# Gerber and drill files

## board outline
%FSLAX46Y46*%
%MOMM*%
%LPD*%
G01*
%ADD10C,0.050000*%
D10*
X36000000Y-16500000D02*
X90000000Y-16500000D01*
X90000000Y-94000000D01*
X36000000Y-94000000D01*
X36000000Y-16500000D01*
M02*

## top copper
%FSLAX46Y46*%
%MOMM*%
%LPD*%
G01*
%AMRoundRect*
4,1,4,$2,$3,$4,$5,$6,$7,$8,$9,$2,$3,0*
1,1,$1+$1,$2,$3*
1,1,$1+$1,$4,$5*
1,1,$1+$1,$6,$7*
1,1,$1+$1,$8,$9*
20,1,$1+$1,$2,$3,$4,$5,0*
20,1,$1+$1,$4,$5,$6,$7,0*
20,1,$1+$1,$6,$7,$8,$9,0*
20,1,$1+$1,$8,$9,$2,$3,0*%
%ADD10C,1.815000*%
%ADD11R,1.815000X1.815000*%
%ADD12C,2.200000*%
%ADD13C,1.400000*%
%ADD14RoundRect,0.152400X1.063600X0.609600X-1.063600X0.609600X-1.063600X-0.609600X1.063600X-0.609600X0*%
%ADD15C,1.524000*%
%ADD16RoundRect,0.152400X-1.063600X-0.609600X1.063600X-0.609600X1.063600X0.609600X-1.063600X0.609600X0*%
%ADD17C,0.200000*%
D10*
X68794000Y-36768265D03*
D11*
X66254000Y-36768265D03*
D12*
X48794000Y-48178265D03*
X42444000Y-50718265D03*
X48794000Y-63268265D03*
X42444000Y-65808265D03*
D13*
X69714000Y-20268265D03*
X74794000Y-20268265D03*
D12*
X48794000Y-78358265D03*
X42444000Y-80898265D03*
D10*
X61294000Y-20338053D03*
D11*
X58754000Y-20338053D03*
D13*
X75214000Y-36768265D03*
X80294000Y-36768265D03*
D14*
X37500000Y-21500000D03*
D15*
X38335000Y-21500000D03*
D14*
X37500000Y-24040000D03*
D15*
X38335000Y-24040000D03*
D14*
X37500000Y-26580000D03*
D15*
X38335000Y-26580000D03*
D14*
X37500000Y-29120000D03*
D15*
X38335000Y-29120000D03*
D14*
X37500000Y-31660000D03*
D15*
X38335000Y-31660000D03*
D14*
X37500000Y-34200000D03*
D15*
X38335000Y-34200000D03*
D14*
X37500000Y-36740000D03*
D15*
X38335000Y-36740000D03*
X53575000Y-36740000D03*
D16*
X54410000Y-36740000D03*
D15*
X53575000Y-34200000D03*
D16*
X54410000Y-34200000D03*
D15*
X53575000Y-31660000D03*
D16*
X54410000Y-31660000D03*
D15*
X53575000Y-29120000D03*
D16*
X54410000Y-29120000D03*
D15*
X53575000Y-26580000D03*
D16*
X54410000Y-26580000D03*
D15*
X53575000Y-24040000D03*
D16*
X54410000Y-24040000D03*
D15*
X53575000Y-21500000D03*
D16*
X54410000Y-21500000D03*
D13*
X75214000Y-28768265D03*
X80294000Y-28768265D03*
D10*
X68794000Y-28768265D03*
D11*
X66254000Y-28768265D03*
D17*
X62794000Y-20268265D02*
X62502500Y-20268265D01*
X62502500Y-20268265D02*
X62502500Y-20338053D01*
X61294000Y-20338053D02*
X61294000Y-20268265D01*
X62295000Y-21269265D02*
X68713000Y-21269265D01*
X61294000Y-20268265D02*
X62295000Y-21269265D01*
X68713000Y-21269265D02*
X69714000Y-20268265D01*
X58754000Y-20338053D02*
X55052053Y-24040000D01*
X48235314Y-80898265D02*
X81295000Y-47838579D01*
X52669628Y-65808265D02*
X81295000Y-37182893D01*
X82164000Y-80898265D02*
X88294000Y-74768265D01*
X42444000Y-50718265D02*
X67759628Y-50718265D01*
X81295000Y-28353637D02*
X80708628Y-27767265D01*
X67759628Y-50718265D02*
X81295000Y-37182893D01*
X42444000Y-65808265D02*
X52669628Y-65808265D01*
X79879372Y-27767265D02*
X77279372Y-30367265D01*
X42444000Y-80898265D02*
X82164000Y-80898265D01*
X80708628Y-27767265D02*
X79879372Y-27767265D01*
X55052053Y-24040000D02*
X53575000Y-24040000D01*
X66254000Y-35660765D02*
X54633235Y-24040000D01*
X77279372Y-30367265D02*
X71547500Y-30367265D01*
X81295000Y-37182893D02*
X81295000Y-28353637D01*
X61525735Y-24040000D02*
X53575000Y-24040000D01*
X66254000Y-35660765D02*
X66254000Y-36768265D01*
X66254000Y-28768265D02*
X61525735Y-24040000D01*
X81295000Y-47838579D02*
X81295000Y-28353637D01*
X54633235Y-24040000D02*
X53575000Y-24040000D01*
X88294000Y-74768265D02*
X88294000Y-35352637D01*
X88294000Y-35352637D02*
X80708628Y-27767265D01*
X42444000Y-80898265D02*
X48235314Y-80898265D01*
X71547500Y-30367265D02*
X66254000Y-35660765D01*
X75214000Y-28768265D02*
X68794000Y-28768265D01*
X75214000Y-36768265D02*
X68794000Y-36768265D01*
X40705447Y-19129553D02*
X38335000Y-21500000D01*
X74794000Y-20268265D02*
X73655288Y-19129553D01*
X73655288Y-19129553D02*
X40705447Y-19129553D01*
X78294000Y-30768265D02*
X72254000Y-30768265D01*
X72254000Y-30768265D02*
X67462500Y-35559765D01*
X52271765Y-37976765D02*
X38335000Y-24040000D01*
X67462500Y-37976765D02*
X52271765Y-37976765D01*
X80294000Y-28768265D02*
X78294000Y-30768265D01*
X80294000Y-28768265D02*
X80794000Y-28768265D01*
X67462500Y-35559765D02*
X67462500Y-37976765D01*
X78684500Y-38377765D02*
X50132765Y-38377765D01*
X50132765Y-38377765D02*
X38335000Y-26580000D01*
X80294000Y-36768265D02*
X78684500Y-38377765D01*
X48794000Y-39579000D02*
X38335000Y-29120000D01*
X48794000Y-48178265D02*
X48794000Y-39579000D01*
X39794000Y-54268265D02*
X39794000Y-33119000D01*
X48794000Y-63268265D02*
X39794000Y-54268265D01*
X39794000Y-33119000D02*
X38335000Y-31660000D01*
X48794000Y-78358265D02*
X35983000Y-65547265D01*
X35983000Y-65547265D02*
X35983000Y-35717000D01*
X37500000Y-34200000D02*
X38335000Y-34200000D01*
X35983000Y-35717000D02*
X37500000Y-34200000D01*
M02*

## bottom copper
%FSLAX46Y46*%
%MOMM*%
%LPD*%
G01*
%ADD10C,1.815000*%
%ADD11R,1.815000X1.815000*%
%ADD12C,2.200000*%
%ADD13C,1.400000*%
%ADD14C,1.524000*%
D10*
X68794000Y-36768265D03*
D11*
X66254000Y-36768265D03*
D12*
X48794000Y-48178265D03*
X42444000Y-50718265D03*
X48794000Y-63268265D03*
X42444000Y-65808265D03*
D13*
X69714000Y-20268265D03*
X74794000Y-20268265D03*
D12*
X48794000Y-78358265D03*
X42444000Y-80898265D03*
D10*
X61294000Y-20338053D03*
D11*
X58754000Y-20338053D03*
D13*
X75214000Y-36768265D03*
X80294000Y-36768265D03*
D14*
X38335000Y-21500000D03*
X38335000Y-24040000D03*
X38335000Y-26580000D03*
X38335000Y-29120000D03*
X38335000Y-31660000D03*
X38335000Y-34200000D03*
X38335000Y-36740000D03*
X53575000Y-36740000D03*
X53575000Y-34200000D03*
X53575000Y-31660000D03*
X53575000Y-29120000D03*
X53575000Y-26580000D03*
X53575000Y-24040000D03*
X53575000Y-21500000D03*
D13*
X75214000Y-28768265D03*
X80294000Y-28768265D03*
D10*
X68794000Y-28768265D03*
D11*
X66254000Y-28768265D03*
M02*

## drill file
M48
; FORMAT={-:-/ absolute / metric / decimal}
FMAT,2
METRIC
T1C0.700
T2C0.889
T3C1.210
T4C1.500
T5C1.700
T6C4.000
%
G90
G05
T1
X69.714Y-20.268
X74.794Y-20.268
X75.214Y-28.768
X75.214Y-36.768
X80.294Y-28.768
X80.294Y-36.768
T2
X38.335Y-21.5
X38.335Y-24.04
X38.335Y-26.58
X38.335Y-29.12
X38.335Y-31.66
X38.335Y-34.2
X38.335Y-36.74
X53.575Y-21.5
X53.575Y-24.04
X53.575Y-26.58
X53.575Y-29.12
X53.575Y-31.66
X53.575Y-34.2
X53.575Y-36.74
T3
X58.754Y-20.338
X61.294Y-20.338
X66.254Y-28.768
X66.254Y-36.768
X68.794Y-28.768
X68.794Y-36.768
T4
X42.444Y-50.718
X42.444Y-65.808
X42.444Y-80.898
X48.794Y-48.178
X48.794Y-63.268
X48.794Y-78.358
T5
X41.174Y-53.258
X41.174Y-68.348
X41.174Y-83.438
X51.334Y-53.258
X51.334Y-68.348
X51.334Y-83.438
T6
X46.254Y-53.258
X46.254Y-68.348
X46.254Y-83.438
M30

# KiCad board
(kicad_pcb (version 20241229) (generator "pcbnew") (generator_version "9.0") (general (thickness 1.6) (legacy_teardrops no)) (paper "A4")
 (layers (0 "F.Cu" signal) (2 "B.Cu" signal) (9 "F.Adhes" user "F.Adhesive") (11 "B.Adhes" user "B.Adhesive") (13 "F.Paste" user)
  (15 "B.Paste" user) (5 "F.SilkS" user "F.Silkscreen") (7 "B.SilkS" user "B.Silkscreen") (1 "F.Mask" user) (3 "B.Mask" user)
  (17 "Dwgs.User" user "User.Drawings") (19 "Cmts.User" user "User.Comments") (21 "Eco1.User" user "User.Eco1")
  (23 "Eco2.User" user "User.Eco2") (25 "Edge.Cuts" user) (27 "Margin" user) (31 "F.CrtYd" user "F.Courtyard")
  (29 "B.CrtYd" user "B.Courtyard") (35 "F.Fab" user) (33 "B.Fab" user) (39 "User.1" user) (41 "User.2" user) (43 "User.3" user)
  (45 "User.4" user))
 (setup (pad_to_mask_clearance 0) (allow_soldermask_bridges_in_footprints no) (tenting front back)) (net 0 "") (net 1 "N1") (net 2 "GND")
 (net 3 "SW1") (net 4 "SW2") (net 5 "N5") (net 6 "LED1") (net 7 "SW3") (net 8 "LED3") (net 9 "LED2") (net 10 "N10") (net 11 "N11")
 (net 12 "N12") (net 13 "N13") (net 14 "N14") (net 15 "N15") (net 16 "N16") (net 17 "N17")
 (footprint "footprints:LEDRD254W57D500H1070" (layer "F.Cu") (at 67.524 36.768265)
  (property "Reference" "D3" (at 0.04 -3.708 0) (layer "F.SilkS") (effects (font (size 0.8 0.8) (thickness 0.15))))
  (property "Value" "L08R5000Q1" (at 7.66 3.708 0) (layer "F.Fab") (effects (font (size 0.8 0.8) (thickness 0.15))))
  (pad "A" thru_hole circle (at 1.27 0) (size 1.815 1.815) (drill 1.21) (layers "*.Cu" "*.Mask") (remove_unused_layers no) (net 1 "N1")
   (solder_mask_margin 0.102))
  (pad "C" thru_hole rect (at -1.27 0) (size 1.815 1.815) (drill 1.21) (layers "*.Cu" "*.Mask") (remove_unused_layers no) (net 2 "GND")
   (solder_mask_margin 0.102)))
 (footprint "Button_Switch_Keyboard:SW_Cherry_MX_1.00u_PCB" (layer "F.Cu") (at 48.794 48.178265)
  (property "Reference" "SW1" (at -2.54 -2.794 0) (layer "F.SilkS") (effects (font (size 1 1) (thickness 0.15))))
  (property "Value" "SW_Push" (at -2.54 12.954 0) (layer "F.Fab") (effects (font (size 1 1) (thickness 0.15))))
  (pad "" np_thru_hole circle (at -7.62 5.08) (size 1.7 1.7) (drill 1.7) (layers "*.Cu" "*.Mask"))
  (pad "" np_thru_hole circle (at -2.54 5.08) (size 4 4) (drill 4) (layers "*.Cu" "*.Mask"))
  (pad "" np_thru_hole circle (at 2.54 5.08) (size 1.7 1.7) (drill 1.7) (layers "*.Cu" "*.Mask"))
  (pad "1" thru_hole circle (at 0 0) (size 2.2 2.2) (drill 1.5) (layers "*.Cu" "*.Mask") (remove_unused_layers no) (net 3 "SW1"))
  (pad "2" thru_hole circle (at -6.35 2.54) (size 2.2 2.2) (drill 1.5) (layers "*.Cu" "*.Mask") (remove_unused_layers no) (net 2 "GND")))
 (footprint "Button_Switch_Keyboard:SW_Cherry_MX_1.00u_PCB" (layer "F.Cu") (at 48.794 63.268265)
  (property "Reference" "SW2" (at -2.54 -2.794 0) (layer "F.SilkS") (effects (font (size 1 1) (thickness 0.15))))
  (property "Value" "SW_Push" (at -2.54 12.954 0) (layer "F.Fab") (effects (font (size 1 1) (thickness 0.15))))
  (pad "" np_thru_hole circle (at -7.62 5.08) (size 1.7 1.7) (drill 1.7) (layers "*.Cu" "*.Mask"))
  (pad "" np_thru_hole circle (at -2.54 5.08) (size 4 4) (drill 4) (layers "*.Cu" "*.Mask"))
  (pad "" np_thru_hole circle (at 2.54 5.08) (size 1.7 1.7) (drill 1.7) (layers "*.Cu" "*.Mask"))
  (pad "1" thru_hole circle (at 0 0) (size 2.2 2.2) (drill 1.5) (layers "*.Cu" "*.Mask") (remove_unused_layers no) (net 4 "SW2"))
  (pad "2" thru_hole circle (at -6.35 2.54) (size 2.2 2.2) (drill 1.5) (layers "*.Cu" "*.Mask") (remove_unused_layers no) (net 2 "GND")))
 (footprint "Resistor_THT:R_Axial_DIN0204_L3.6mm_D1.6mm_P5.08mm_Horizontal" (layer "F.Cu") (at 69.714 20.268265)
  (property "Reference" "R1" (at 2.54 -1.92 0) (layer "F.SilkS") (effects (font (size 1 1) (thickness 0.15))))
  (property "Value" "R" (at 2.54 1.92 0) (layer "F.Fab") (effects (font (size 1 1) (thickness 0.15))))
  (pad "1" thru_hole circle (at 0 0) (size 1.4 1.4) (drill 0.7) (layers "*.Cu" "*.Mask") (remove_unused_layers no) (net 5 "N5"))
  (pad "2" thru_hole circle (at 5.08 0) (size 1.4 1.4) (drill 0.7) (layers "*.Cu" "*.Mask") (remove_unused_layers no) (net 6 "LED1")))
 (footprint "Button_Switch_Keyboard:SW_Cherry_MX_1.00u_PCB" (layer "F.Cu") (at 48.794 78.358265)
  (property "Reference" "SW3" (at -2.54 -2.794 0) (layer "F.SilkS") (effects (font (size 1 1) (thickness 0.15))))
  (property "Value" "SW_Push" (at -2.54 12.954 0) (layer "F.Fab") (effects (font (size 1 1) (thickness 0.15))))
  (pad "" np_thru_hole circle (at -7.62 5.08) (size 1.7 1.7) (drill 1.7) (layers "*.Cu" "*.Mask"))
  (pad "" np_thru_hole circle (at -2.54 5.08) (size 4 4) (drill 4) (layers "*.Cu" "*.Mask"))
  (pad "" np_thru_hole circle (at 2.54 5.08) (size 1.7 1.7) (drill 1.7) (layers "*.Cu" "*.Mask"))
  (pad "1" thru_hole circle (at 0 0) (size 2.2 2.2) (drill 1.5) (layers "*.Cu" "*.Mask") (remove_unused_layers no) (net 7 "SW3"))
  (pad "2" thru_hole circle (at -6.35 2.54) (size 2.2 2.2) (drill 1.5) (layers "*.Cu" "*.Mask") (remove_unused_layers no) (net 2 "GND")))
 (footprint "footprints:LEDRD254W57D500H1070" (layer "F.Cu") (at 60.024 20.338053)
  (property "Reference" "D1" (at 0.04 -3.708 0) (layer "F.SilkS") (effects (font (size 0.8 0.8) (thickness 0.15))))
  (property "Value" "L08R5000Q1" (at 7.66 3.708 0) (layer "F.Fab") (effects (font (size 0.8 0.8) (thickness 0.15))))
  (pad "A" thru_hole circle (at 1.27 0) (size 1.815 1.815) (drill 1.21) (layers "*.Cu" "*.Mask") (remove_unused_layers no) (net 5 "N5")
   (solder_mask_margin 0.102))
  (pad "C" thru_hole rect (at -1.27 0) (size 1.815 1.815) (drill 1.21) (layers "*.Cu" "*.Mask") (remove_unused_layers no) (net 2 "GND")
   (solder_mask_margin 0.102)))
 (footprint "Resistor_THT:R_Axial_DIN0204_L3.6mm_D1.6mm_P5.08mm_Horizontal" (layer "F.Cu") (at 75.214 36.768265)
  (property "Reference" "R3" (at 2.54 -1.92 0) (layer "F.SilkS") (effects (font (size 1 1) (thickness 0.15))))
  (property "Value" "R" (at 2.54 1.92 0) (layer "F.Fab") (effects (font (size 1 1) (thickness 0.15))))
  (pad "1" thru_hole circle (at 0 0) (size 1.4 1.4) (drill 0.7) (layers "*.Cu" "*.Mask") (remove_unused_layers no) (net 1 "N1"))
  (pad "2" thru_hole circle (at 5.08 0) (size 1.4 1.4) (drill 0.7) (layers "*.Cu" "*.Mask") (remove_unused_layers no) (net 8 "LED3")))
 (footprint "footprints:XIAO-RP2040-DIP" (layer "F.Cu") (at 45.955 29.12)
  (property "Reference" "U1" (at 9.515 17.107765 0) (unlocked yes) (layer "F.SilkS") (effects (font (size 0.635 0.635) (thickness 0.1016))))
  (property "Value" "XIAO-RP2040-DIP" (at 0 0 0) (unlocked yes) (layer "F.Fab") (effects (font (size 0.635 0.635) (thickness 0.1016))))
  (pad "1" smd roundrect (at -8.455 -7.62 180) (size 2.432 1.524) (layers "F.Cu" "F.Mask") (roundrect_rratio 0.1) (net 6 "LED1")
   (thermal_bridge_angle 45))
  (pad "1" thru_hole circle (at -7.62 -7.62 180) (size 1.524 1.524) (drill 0.889) (layers "*.Cu" "*.Mask") (remove_unused_layers no)
   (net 6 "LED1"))
  (pad "2" smd roundrect (at -8.455 -5.08 180) (size 2.432 1.524) (layers "F.Cu" "F.Mask") (roundrect_rratio 0.1) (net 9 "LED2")
   (thermal_bridge_angle 45))
  (pad "2" thru_hole circle (at -7.62 -5.08 180) (size 1.524 1.524) (drill 0.889) (layers "*.Cu" "*.Mask") (remove_unused_layers no)
   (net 9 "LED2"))
  (pad "3" smd roundrect (at -8.455 -2.54 180) (size 2.432 1.524) (layers "F.Cu" "F.Mask") (roundrect_rratio 0.1) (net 8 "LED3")
   (thermal_bridge_angle 45))
  (pad "3" thru_hole circle (at -7.62 -2.54 180) (size 1.524 1.524) (drill 0.889) (layers "*.Cu" "*.Mask") (remove_unused_layers no)
   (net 8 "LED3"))
  (pad "4" smd roundrect (at -8.455 0 180) (size 2.432 1.524) (layers "F.Cu" "F.Mask") (roundrect_rratio 0.1) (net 3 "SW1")
   (thermal_bridge_angle 45))
  (pad "4" thru_hole circle (at -7.62 0 180) (size 1.524 1.524) (drill 0.889) (layers "*.Cu" "*.Mask") (remove_unused_layers no)
   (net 3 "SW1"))
  (pad "5" smd roundrect (at -8.455 2.54 180) (size 2.432 1.524) (layers "F.Cu" "F.Mask") (roundrect_rratio 0.1) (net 4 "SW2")
   (thermal_bridge_angle 45))
  (pad "5" thru_hole circle (at -7.62 2.54 180) (size 1.524 1.524) (drill 0.889) (layers "*.Cu" "*.Mask") (remove_unused_layers no)
   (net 4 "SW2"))
  (pad "6" smd roundrect (at -8.455 5.08 180) (size 2.432 1.524) (layers "F.Cu" "F.Mask") (roundrect_rratio 0.1) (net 7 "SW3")
   (thermal_bridge_angle 45))
  (pad "6" thru_hole circle (at -7.62 5.08 180) (size 1.524 1.524) (drill 0.889) (layers "*.Cu" "*.Mask") (remove_unused_layers no)
   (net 7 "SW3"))
  (pad "7" smd roundrect (at -8.455 7.62 180) (size 2.432 1.524) (layers "F.Cu" "F.Mask") (roundrect_rratio 0.1) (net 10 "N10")
   (thermal_bridge_angle 45))
  (pad "7" thru_hole circle (at -7.62 7.62 180) (size 1.524 1.524) (drill 0.889) (layers "*.Cu" "*.Mask") (remove_unused_layers no)
   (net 10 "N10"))
  (pad "8" thru_hole circle (at 7.62 7.62) (size 1.524 1.524) (drill 0.889) (layers "*.Cu" "*.Mask") (remove_unused_layers no)
   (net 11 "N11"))
  (pad "8" smd roundrect (at 8.455 7.62) (size 2.432 1.524) (layers "F.Cu" "F.Mask") (roundrect_rratio 0.1) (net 11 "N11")
   (thermal_bridge_angle 45))
  (pad "9" thru_hole circle (at 7.62 5.08) (size 1.524 1.524) (drill 0.889) (layers "*.Cu" "*.Mask") (remove_unused_layers no)
   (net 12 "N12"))
  (pad "9" smd roundrect (at 8.455 5.08) (size 2.432 1.524) (layers "F.Cu" "F.Mask") (roundrect_rratio 0.1) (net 12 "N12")
   (thermal_bridge_angle 45))
  (pad "10" thru_hole circle (at 7.62 2.54) (size 1.524 1.524) (drill 0.889) (layers "*.Cu" "*.Mask") (remove_unused_layers no)
   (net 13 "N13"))
  (pad "10" smd roundrect (at 8.455 2.54) (size 2.432 1.524) (layers "F.Cu" "F.Mask") (roundrect_rratio 0.1) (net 13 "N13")
   (thermal_bridge_angle 45))
  (pad "11" thru_hole circle (at 7.62 0) (size 1.524 1.524) (drill 0.889) (layers "*.Cu" "*.Mask") (remove_unused_layers no) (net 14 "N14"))
  (pad "11" smd roundrect (at 8.455 0) (size 2.432 1.524) (layers "F.Cu" "F.Mask") (roundrect_rratio 0.1) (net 14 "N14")
   (thermal_bridge_angle 45))
  (pad "12" thru_hole circle (at 7.62 -2.54) (size 1.524 1.524) (drill 0.889) (layers "*.Cu" "*.Mask") (remove_unused_layers no)
   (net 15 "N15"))
  (pad "12" smd roundrect (at 8.455 -2.54) (size 2.432 1.524) (layers "F.Cu" "F.Mask") (roundrect_rratio 0.1) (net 15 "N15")
   (thermal_bridge_angle 45))
  (pad "13" thru_hole circle (at 7.62 -5.08) (size 1.524 1.524) (drill 0.889) (layers "*.Cu" "*.Mask") (remove_unused_layers no)
   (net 2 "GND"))
  (pad "13" smd roundrect (at 8.455 -5.08) (size 2.432 1.524) (layers "F.Cu" "F.Mask") (roundrect_rratio 0.1) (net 2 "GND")
   (thermal_bridge_angle 45))
  (pad "14" thru_hole circle (at 7.62 -7.62) (size 1.524 1.524) (drill 0.889) (layers "*.Cu" "*.Mask") (remove_unused_layers no)
   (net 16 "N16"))
  (pad "14" smd roundrect (at 8.455 -7.62) (size 2.432 1.524) (layers "F.Cu" "F.Mask") (roundrect_rratio 0.1) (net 16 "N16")
   (thermal_bridge_angle 45)))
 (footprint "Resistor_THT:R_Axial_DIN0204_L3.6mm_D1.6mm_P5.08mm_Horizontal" (layer "F.Cu") (at 75.214 28.768265)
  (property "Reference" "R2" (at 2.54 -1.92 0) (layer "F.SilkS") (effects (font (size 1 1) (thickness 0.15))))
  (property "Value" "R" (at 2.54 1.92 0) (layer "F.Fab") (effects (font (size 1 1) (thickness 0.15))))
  (pad "1" thru_hole circle (at 0 0) (size 1.4 1.4) (drill 0.7) (layers "*.Cu" "*.Mask") (remove_unused_layers no) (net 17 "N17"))
  (pad "2" thru_hole circle (at 5.08 0) (size 1.4 1.4) (drill 0.7) (layers "*.Cu" "*.Mask") (remove_unused_layers no) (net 9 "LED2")))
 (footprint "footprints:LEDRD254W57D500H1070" (layer "F.Cu") (at 67.524 28.768265)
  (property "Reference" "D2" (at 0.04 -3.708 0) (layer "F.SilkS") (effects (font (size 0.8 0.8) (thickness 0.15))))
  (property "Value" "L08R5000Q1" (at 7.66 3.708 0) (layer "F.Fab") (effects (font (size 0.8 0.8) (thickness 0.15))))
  (pad "A" thru_hole circle (at 1.27 0) (size 1.815 1.815) (drill 1.21) (layers "*.Cu" "*.Mask") (remove_unused_layers no) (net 17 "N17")
   (solder_mask_margin 0.102))
  (pad "C" thru_hole rect (at -1.27 0) (size 1.815 1.815) (drill 1.21) (layers "*.Cu" "*.Mask") (remove_unused_layers no) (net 2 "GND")
   (solder_mask_margin 0.102)))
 (gr_rect (start 36 16.5) (end 90 94) (stroke (width 0.05) (type default)) (fill no) (layer "Edge.Cuts"))
 (segment (start 62.794 20.268265) (end 62.5025 20.268265) (width 0.2) (layer "F.Cu") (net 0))
 (segment (start 62.5025 20.268265) (end 62.5025 20.338053) (width 0.2) (layer "F.Cu") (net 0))
 (segment (start 61.294 20.338053) (end 61.294 20.268265) (width 0.2) (layer "F.Cu") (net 5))
 (segment (start 62.295 21.269265) (end 68.713 21.269265) (width 0.2) (layer "F.Cu") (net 5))
 (segment (start 61.294 20.268265) (end 62.295 21.269265) (width 0.2) (layer "F.Cu") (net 5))
 (segment (start 68.713 21.269265) (end 69.714 20.268265) (width 0.2) (layer "F.Cu") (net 5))
 (segment (start 58.754 20.338053) (end 55.052053 24.04) (width 0.2) (layer "F.Cu") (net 2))
 (segment (start 48.235314 80.898265) (end 81.295 47.838579) (width 0.2) (layer "F.Cu") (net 2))
 (segment (start 52.669628 65.808265) (end 81.295 37.182893) (width 0.2) (layer "F.Cu") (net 2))
 (segment (start 82.164 80.898265) (end 88.294 74.768265) (width 0.2) (layer "F.Cu") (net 2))
 (segment (start 42.444 50.718265) (end 67.759628 50.718265) (width 0.2) (layer "F.Cu") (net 2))
 (segment (start 81.295 28.353637) (end 80.708628 27.767265) (width 0.2) (layer "F.Cu") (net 2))
 (segment (start 67.759628 50.718265) (end 81.295 37.182893) (width 0.2) (layer "F.Cu") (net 2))
 (segment (start 42.444 65.808265) (end 52.669628 65.808265) (width 0.2) (layer "F.Cu") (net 2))
 (segment (start 79.879372 27.767265) (end 77.279372 30.367265) (width 0.2) (layer "F.Cu") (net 2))
 (segment (start 42.444 80.898265) (end 82.164 80.898265) (width 0.2) (layer "F.Cu") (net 2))
 (segment (start 80.708628 27.767265) (end 79.879372 27.767265) (width 0.2) (layer "F.Cu") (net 2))
 (segment (start 55.052053 24.04) (end 53.575 24.04) (width 0.2) (layer "F.Cu") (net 2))
 (segment (start 66.254 35.660765) (end 54.633235 24.04) (width 0.2) (layer "F.Cu") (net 2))
 (segment (start 77.279372 30.367265) (end 71.5475 30.367265) (width 0.2) (layer "F.Cu") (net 2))
 (segment (start 81.295 37.182893) (end 81.295 28.353637) (width 0.2) (layer "F.Cu") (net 2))
 (segment (start 61.525735 24.04) (end 53.575 24.04) (width 0.2) (layer "F.Cu") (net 2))
 (segment (start 66.254 35.660765) (end 66.254 36.768265) (width 0.2) (layer "F.Cu") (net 2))
 (segment (start 66.254 28.768265) (end 61.525735 24.04) (width 0.2) (layer "F.Cu") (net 2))
 (segment (start 81.295 47.838579) (end 81.295 28.353637) (width 0.2) (layer "F.Cu") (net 2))
 (segment (start 54.633235 24.04) (end 53.575 24.04) (width 0.2) (layer "F.Cu") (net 2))
 (segment (start 88.294 74.768265) (end 88.294 35.352637) (width 0.2) (layer "F.Cu") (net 2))
 (segment (start 88.294 35.352637) (end 80.708628 27.767265) (width 0.2) (layer "F.Cu") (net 2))
 (segment (start 42.444 80.898265) (end 48.235314 80.898265) (width 0.2) (layer "F.Cu") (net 2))
 (segment (start 71.5475 30.367265) (end 66.254 35.660765) (width 0.2) (layer "F.Cu") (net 2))
 (segment (start 75.214 28.768265) (end 68.794 28.768265) (width 0.2) (layer "F.Cu") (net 17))
 (segment (start 75.214 36.768265) (end 68.794 36.768265) (width 0.2) (layer "F.Cu") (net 1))
 (segment (start 40.705447 19.129553) (end 38.335 21.5) (width 0.2) (layer "F.Cu") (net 6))
 (segment (start 74.794 20.268265) (end 73.655288 19.129553) (width 0.2) (layer "F.Cu") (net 6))
 (segment (start 73.655288 19.129553) (end 40.705447 19.129553) (width 0.2) (layer "F.Cu") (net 6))
 (segment (start 78.294 30.768265) (end 72.254 30.768265) (width 0.2) (layer "F.Cu") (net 9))
 (segment (start 72.254 30.768265) (end 67.4625 35.559765) (width 0.2) (layer "F.Cu") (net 9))
 (segment (start 52.271765 37.976765) (end 38.335 24.04) (width 0.2) (layer "F.Cu") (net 9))
 (segment (start 67.4625 37.976765) (end 52.271765 37.976765) (width 0.2) (layer "F.Cu") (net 9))
 (segment (start 80.294 28.768265) (end 78.294 30.768265) (width 0.2) (layer "F.Cu") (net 9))
 (segment (start 80.294 28.768265) (end 80.794 28.768265) (width 0.2) (layer "F.Cu") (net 9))
 (segment (start 67.4625 35.559765) (end 67.4625 37.976765) (width 0.2) (layer "F.Cu") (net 9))
 (segment (start 78.6845 38.377765) (end 50.132765 38.377765) (width 0.2) (layer "F.Cu") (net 8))
 (segment (start 50.132765 38.377765) (end 38.335 26.58) (width 0.2) (layer "F.Cu") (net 8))
 (segment (start 80.294 36.768265) (end 78.6845 38.377765) (width 0.2) (layer "F.Cu") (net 8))
 (segment (start 48.794 39.579) (end 38.335 29.12) (width 0.2) (layer "F.Cu") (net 3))
 (segment (start 48.794 48.178265) (end 48.794 39.579) (width 0.2) (layer "F.Cu") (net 3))
 (segment (start 39.794 54.268265) (end 39.794 33.119) (width 0.2) (layer "F.Cu") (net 4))
 (segment (start 48.794 63.268265) (end 39.794 54.268265) (width 0.2) (layer "F.Cu") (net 4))
 (segment (start 39.794 33.119) (end 38.335 31.66) (width 0.2) (layer "F.Cu") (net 4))
 (segment (start 48.794 78.358265) (end 35.983 65.547265) (width 0.2) (layer "F.Cu") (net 7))
 (segment (start 35.983 65.547265) (end 35.983 35.717) (width 0.2) (layer "F.Cu") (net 7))
 (segment (start 37.5 34.2) (end 38.335 34.2) (width 0.2) (layer "F.Cu") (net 7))
 (segment (start 35.983 35.717) (end 37.5 34.2) (width 0.2) (layer "F.Cu") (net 7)))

